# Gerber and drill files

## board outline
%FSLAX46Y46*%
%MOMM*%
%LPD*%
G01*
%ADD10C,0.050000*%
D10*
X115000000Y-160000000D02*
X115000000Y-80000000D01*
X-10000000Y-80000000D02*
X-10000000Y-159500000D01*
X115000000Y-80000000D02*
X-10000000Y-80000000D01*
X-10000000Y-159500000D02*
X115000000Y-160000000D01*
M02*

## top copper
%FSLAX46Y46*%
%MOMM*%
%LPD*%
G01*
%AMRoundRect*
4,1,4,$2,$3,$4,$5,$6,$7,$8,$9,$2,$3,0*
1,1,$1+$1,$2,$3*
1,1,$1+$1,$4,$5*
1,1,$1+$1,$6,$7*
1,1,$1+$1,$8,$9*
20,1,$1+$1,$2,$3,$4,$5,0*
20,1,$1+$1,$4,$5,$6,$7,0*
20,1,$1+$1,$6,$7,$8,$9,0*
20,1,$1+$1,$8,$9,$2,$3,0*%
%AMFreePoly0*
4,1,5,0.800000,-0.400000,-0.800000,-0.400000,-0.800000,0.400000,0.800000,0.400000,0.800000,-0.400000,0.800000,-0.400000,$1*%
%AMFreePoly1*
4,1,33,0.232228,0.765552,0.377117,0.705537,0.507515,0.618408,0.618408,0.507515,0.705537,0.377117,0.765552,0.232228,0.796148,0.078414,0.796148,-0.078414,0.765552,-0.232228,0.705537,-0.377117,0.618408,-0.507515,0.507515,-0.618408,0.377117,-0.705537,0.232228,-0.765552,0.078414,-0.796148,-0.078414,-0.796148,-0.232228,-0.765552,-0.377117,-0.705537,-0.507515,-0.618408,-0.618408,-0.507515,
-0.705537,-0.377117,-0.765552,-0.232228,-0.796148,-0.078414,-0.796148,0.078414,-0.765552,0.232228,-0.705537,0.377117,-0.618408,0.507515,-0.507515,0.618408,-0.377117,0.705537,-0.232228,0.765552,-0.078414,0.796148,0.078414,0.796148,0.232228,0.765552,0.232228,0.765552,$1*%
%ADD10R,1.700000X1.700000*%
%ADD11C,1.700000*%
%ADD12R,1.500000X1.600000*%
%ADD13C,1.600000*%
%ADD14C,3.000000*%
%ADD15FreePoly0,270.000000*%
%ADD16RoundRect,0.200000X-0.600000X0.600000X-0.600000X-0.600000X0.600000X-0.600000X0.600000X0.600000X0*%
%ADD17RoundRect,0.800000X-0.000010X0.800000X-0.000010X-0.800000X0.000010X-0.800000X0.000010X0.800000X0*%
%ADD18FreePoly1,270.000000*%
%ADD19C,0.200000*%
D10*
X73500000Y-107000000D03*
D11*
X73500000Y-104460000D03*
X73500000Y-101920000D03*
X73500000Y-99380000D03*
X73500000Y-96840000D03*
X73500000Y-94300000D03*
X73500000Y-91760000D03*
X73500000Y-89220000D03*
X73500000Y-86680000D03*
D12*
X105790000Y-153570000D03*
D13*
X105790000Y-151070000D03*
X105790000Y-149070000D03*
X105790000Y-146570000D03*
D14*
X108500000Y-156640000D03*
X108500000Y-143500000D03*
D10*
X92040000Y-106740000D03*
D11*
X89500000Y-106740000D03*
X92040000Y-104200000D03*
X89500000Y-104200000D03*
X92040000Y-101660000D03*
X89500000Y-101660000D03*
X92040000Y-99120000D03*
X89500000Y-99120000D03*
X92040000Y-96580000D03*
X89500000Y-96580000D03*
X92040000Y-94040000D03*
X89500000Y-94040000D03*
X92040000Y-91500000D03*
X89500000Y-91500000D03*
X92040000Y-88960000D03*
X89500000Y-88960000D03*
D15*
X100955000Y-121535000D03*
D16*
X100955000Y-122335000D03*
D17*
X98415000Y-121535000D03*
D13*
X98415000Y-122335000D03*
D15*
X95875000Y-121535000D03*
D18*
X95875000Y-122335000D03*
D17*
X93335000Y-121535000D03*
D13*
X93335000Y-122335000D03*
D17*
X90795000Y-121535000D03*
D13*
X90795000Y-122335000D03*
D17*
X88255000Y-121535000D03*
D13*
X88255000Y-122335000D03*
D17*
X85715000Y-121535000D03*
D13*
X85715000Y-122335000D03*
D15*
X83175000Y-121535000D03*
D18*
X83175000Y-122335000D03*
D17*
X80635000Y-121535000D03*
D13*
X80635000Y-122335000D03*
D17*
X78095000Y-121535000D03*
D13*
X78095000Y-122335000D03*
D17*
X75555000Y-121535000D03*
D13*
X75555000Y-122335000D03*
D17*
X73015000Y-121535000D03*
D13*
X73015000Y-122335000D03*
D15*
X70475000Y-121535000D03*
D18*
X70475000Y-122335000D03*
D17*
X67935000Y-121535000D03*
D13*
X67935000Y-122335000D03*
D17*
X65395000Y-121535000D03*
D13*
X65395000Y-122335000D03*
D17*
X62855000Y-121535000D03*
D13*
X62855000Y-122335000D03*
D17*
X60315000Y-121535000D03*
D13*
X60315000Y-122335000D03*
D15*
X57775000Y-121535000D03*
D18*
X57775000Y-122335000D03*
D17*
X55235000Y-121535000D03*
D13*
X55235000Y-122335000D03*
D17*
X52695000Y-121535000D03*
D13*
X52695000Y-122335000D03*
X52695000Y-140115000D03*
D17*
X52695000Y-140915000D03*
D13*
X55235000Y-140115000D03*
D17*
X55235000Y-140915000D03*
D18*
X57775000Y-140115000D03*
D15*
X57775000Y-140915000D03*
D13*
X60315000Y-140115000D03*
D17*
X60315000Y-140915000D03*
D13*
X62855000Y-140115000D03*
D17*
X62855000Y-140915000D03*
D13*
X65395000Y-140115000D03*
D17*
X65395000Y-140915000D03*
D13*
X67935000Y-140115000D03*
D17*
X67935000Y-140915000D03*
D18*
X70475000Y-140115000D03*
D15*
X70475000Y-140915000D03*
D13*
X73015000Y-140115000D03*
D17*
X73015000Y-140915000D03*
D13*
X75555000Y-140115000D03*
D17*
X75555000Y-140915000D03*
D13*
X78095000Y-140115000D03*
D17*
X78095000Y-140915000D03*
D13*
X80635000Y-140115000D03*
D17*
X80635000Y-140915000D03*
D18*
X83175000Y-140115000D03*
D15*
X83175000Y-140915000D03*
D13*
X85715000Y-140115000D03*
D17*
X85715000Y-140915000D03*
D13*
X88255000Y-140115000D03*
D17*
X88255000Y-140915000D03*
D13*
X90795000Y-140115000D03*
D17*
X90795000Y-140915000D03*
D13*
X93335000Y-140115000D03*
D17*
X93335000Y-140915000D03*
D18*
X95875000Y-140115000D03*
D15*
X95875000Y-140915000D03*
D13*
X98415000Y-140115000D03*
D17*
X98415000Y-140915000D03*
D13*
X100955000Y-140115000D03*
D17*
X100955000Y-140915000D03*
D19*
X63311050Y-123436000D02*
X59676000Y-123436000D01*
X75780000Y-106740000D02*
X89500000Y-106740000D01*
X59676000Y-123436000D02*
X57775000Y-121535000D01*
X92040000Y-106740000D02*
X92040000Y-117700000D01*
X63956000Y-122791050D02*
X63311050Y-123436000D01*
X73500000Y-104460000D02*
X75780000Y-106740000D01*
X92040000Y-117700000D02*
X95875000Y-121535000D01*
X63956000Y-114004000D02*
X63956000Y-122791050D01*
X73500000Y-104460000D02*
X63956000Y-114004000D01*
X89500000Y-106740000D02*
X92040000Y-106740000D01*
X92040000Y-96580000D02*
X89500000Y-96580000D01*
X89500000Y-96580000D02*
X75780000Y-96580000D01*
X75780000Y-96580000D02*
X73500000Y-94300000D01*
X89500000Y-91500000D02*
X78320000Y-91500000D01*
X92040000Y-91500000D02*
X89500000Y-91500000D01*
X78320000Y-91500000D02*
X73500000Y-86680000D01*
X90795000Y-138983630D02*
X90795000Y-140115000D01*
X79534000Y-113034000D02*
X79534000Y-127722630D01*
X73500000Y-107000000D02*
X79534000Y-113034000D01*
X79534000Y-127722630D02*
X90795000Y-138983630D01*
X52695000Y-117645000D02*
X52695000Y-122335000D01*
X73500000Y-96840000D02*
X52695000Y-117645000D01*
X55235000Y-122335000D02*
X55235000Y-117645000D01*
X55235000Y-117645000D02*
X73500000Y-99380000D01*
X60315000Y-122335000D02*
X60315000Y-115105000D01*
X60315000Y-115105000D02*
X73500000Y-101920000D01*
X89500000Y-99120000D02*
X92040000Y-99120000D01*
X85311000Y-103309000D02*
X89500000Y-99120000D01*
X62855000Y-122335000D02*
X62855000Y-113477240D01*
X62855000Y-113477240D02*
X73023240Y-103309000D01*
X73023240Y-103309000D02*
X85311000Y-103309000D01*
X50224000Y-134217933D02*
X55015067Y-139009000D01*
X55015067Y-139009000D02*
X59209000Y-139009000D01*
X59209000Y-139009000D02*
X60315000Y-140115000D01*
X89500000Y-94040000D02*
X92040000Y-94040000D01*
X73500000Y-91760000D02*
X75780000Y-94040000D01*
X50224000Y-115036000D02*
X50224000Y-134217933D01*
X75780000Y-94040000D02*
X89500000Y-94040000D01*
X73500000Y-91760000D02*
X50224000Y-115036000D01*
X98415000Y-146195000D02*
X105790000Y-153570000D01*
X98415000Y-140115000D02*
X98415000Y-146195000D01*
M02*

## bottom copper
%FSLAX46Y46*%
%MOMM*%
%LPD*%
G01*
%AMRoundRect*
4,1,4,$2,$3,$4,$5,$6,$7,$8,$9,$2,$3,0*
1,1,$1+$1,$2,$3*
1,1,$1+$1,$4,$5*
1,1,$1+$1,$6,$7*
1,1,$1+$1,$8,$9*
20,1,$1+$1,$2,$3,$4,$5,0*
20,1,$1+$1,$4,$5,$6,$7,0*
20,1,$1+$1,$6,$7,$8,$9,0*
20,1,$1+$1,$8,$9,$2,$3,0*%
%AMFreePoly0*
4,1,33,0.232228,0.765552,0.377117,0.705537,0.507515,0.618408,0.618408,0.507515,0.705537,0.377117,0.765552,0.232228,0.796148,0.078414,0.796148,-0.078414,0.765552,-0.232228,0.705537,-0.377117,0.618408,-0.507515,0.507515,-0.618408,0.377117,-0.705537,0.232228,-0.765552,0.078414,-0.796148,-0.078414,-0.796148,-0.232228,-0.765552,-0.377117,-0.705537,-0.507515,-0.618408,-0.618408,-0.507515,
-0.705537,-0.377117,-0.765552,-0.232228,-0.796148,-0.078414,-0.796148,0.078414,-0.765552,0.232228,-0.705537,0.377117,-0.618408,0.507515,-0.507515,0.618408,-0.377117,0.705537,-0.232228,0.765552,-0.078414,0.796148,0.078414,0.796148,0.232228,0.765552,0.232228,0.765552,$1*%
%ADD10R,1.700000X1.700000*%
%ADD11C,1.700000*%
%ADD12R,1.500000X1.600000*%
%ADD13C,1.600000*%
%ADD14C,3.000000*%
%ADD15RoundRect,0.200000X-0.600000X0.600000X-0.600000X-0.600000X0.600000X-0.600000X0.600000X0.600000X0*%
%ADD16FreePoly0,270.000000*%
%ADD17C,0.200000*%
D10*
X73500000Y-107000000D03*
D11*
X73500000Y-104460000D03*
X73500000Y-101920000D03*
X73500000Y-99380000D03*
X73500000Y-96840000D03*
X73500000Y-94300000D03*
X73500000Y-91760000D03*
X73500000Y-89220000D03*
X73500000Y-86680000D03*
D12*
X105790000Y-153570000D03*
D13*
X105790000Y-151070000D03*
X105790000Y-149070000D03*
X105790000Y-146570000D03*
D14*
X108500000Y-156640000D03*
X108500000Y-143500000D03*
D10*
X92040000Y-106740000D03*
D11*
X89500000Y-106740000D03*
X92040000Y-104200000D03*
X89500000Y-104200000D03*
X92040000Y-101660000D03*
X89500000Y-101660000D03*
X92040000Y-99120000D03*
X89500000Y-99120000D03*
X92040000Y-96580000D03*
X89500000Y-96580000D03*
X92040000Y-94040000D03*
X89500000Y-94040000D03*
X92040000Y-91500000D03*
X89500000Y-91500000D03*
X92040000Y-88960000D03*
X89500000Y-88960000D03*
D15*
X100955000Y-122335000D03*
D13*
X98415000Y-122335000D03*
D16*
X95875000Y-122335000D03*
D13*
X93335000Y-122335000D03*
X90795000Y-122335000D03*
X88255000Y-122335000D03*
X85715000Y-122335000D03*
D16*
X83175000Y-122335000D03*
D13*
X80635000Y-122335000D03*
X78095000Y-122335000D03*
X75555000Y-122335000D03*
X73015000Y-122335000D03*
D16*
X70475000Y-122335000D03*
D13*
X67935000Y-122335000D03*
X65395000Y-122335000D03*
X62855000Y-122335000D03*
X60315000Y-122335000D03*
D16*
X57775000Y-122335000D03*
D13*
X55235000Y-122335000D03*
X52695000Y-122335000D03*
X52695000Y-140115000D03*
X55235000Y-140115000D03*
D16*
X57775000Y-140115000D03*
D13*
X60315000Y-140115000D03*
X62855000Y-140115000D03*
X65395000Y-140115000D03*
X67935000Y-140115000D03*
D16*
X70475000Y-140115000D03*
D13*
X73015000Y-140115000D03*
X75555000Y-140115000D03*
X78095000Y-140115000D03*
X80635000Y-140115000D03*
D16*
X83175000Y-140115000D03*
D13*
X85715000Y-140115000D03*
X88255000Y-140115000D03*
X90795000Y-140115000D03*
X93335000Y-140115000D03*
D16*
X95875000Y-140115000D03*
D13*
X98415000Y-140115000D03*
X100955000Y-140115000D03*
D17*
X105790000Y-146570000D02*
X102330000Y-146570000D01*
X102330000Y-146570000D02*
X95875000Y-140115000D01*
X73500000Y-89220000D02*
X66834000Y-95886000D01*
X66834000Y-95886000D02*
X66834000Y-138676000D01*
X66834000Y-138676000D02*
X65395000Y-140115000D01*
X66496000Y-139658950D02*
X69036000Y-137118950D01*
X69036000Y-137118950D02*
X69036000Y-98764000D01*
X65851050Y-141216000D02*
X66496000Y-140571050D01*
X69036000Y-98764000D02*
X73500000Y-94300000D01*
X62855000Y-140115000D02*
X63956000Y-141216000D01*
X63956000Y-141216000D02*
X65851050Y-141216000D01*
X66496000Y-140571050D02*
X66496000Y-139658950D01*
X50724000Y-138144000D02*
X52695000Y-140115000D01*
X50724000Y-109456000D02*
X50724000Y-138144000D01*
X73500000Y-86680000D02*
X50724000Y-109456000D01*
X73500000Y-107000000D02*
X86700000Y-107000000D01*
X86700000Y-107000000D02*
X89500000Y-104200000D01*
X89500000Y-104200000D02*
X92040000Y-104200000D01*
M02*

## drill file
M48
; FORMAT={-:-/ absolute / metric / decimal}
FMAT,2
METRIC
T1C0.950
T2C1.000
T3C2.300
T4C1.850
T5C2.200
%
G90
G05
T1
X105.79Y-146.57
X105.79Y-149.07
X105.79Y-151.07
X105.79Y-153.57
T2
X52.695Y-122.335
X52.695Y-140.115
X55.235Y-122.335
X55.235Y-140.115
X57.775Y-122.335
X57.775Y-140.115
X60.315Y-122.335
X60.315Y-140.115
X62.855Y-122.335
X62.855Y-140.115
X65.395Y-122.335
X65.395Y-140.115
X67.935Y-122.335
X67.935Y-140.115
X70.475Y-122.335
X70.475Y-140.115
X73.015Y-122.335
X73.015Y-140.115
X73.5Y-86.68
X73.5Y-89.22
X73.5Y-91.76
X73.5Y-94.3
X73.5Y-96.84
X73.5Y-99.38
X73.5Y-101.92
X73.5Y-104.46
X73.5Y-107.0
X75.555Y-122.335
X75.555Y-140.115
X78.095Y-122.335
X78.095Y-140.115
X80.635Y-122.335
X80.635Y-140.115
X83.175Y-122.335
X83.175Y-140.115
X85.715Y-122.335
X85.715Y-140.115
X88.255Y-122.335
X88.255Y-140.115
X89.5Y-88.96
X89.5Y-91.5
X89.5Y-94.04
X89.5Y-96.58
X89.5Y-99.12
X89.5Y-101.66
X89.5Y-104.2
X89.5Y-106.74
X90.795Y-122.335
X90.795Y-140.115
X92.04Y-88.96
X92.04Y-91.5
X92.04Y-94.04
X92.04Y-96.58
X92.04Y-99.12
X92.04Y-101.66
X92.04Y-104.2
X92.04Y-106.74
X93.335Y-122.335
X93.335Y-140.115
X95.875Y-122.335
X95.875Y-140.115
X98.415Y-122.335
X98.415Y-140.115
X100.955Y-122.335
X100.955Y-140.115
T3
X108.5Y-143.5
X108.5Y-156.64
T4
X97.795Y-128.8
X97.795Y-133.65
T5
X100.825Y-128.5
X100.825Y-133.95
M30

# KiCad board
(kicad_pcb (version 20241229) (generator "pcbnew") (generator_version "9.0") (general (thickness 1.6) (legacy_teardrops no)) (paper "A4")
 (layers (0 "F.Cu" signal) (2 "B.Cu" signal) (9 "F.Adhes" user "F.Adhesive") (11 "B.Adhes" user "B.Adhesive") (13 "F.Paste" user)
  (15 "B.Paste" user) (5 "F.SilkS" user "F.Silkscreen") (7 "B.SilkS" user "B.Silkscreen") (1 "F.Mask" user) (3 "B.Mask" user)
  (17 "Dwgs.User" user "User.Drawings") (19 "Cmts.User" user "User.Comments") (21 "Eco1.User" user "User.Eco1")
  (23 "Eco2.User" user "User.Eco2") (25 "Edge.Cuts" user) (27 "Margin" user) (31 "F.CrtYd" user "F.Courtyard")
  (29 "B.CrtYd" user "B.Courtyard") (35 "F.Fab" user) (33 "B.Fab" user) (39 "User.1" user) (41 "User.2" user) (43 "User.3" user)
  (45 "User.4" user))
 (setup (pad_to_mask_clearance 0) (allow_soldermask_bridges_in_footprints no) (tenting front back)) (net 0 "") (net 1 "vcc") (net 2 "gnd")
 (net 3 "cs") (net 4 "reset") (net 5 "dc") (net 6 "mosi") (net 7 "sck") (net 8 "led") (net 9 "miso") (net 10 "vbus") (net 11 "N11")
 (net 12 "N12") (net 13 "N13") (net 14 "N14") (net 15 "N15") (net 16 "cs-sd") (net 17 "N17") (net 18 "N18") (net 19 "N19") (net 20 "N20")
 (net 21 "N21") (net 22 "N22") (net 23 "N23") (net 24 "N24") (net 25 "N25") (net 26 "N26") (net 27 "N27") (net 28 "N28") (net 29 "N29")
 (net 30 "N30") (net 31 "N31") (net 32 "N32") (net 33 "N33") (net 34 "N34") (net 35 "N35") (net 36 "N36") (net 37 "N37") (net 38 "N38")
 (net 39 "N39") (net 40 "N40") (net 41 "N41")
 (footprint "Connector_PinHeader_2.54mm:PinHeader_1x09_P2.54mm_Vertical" (layer "F.Cu") (at 73.5 107 180)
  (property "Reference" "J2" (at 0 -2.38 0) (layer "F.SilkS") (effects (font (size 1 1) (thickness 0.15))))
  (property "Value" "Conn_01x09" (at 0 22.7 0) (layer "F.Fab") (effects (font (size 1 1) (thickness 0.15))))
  (pad "1" thru_hole rect (at 0 0 180) (size 1.7 1.7) (drill 1) (layers "*.Cu" "*.Mask") (remove_unused_layers no) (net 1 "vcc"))
  (pad "2" thru_hole circle (at 0 2.54 180) (size 1.7 1.7) (drill 1) (layers "*.Cu" "*.Mask") (remove_unused_layers no) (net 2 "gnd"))
  (pad "3" thru_hole circle (at 0 5.08 180) (size 1.7 1.7) (drill 1) (layers "*.Cu" "*.Mask") (remove_unused_layers no) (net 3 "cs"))
  (pad "4" thru_hole circle (at 0 7.62 180) (size 1.7 1.7) (drill 1) (layers "*.Cu" "*.Mask") (remove_unused_layers no) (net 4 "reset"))
  (pad "5" thru_hole circle (at 0 10.16 180) (size 1.7 1.7) (drill 1) (layers "*.Cu" "*.Mask") (remove_unused_layers no) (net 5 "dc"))
  (pad "6" thru_hole circle (at 0 12.7 180) (size 1.7 1.7) (drill 1) (layers "*.Cu" "*.Mask") (remove_unused_layers no) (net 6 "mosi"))
  (pad "7" thru_hole circle (at 0 15.24 180) (size 1.7 1.7) (drill 1) (layers "*.Cu" "*.Mask") (remove_unused_layers no) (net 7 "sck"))
  (pad "8" thru_hole circle (at 0 17.78 180) (size 1.7 1.7) (drill 1) (layers "*.Cu" "*.Mask") (remove_unused_layers no) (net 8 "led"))
  (pad "9" thru_hole circle (at 0 20.32 180) (size 1.7 1.7) (drill 1) (layers "*.Cu" "*.Mask") (remove_unused_layers no) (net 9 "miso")))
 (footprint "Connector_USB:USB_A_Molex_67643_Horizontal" (layer "F.Cu") (at 105.79 153.57 90)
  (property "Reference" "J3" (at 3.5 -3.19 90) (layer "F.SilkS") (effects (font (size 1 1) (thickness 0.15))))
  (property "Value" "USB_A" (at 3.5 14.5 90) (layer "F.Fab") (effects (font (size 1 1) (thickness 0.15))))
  (pad "1" thru_hole rect (at 0 0 90) (size 1.6 1.5) (drill 0.95) (layers "*.Cu" "*.Mask") (remove_unused_layers no) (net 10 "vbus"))
  (pad "2" thru_hole circle (at 2.5 0 90) (size 1.6 1.6) (drill 0.95) (layers "*.Cu" "*.Mask") (remove_unused_layers no) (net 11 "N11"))
  (pad "3" thru_hole circle (at 4.5 0 90) (size 1.6 1.6) (drill 0.95) (layers "*.Cu" "*.Mask") (remove_unused_layers no) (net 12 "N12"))
  (pad "4" thru_hole circle (at 7 0 90) (size 1.6 1.6) (drill 0.95) (layers "*.Cu" "*.Mask") (remove_unused_layers no) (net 2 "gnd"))
  (pad "5" thru_hole circle (at -3.07 2.71 90) (size 3 3) (drill 2.3) (layers "*.Cu" "*.Mask") (remove_unused_layers no) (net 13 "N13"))
  (pad "5" thru_hole circle (at 10.07 2.71 90) (size 3 3) (drill 2.3) (layers "*.Cu" "*.Mask") (remove_unused_layers no) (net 13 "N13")))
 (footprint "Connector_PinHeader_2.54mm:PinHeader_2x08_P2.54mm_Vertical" (layer "F.Cu") (at 92.04 106.74 180)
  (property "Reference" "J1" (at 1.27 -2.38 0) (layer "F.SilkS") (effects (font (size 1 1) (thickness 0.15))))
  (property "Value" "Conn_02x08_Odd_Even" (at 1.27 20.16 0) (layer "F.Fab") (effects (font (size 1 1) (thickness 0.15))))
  (pad "1" thru_hole rect (at 0 0 180) (size 1.7 1.7) (drill 1) (layers "*.Cu" "*.Mask") (remove_unused_layers no) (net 2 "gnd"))
  (pad "2" thru_hole circle (at 2.54 0 180) (size 1.7 1.7) (drill 1) (layers "*.Cu" "*.Mask") (remove_unused_layers no) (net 2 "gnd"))
  (pad "3" thru_hole circle (at 0 2.54 180) (size 1.7 1.7) (drill 1) (layers "*.Cu" "*.Mask") (remove_unused_layers no) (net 1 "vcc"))
  (pad "4" thru_hole circle (at 2.54 2.54 180) (size 1.7 1.7) (drill 1) (layers "*.Cu" "*.Mask") (remove_unused_layers no) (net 1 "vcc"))
  (pad "5" thru_hole circle (at 0 5.08 180) (size 1.7 1.7) (drill 1) (layers "*.Cu" "*.Mask") (remove_unused_layers no) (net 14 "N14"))
  (pad "6" thru_hole circle (at 2.54 5.08 180) (size 1.7 1.7) (drill 1) (layers "*.Cu" "*.Mask") (remove_unused_layers no) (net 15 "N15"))
  (pad "7" thru_hole circle (at 0 7.62 180) (size 1.7 1.7) (drill 1) (layers "*.Cu" "*.Mask") (remove_unused_layers no) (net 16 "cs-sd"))
  (pad "8" thru_hole circle (at 2.54 7.62 180) (size 1.7 1.7) (drill 1) (layers "*.Cu" "*.Mask") (remove_unused_layers no) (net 16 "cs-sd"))
  (pad "9" thru_hole circle (at 0 10.16 180) (size 1.7 1.7) (drill 1) (layers "*.Cu" "*.Mask") (remove_unused_layers no) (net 6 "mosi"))
  (pad "10" thru_hole circle (at 2.54 10.16 180) (size 1.7 1.7) (drill 1) (layers "*.Cu" "*.Mask") (remove_unused_layers no) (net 6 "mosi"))
  (pad "11" thru_hole circle (at 0 12.7 180) (size 1.7 1.7) (drill 1) (layers "*.Cu" "*.Mask") (remove_unused_layers no) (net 7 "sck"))
  (pad "12" thru_hole circle (at 2.54 12.7 180) (size 1.7 1.7) (drill 1) (layers "*.Cu" "*.Mask") (remove_unused_layers no) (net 7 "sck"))
  (pad "13" thru_hole circle (at 0 15.24 180) (size 1.7 1.7) (drill 1) (layers "*.Cu" "*.Mask") (remove_unused_layers no) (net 9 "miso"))
  (pad "14" thru_hole circle (at 2.54 15.24 180) (size 1.7 1.7) (drill 1) (layers "*.Cu" "*.Mask") (remove_unused_layers no) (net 9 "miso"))
  (pad "15" thru_hole circle (at 0 17.78 180) (size 1.7 1.7) (drill 1) (layers "*.Cu" "*.Mask") (remove_unused_layers no) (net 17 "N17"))
  (pad "16" thru_hole circle (at 2.54 17.78 180) (size 1.7 1.7) (drill 1) (layers "*.Cu" "*.Mask") (remove_unused_layers no) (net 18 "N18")))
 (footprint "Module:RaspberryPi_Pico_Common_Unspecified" (layer "F.Cu") (at 76.825 131.225 -90)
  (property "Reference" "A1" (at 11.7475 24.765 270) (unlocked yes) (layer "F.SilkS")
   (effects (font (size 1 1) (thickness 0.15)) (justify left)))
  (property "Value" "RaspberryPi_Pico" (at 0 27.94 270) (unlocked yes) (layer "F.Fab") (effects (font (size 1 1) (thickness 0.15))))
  (pad "" np_thru_hole circle (at -2.725 -24 270) (size 2.2 2.2) (drill 2.2) (layers "*.Mask"))
  (pad "" np_thru_hole circle (at -2.425 -20.97 270) (size 1.85 1.85) (drill 1.85) (layers "*.Mask"))
  (pad "" np_thru_hole circle (at 2.425 -20.97 270) (size 1.85 1.85) (drill 1.85) (layers "*.Mask"))
  (pad "" np_thru_hole circle (at 2.725 -24 270) (size 2.2 2.2) (drill 2.2) (layers "*.Mask"))
  (pad "1" smd custom (at -9.69 -24.13 270) (size 1.6 0.8) (layers "F.Cu" "F.Mask") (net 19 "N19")
   (options (clearance outline) (anchor rect)) (primitives))
  (pad "1" thru_hole roundrect (at -8.89 -24.13 270) (size 1.6 1.6) (drill 1) (layers "*.Cu" "*.Mask") (remove_unused_layers no)
   (roundrect_rratio 0.125) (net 19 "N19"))
  (pad "2" smd roundrect (at -9.69 -21.59 270) (size 3.2 1.6) (layers "F.Cu" "F.Mask") (roundrect_rratio 0.5) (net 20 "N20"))
  (pad "2" thru_hole circle (at -8.89 -21.59 270) (size 1.6 1.6) (drill 1) (layers "*.Cu" "*.Mask") (remove_unused_layers no) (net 20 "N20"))
  (pad "3" smd custom (at -9.69 -19.05 270) (size 1.6 0.8) (layers "F.Cu" "F.Mask") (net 2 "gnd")
   (options (clearance outline) (anchor rect)) (primitives))
  (pad "3" thru_hole custom (at -8.89 -19.05 270) (size 1.6 1.6) (drill 1) (layers "*.Cu" "*.Mask") (remove_unused_layers no) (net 2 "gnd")
   (options (clearance outline) (anchor circle)) (primitives))
  (pad "4" smd roundrect (at -9.69 -16.51 270) (size 3.2 1.6) (layers "F.Cu" "F.Mask") (roundrect_rratio 0.5) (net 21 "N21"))
  (pad "4" thru_hole circle (at -8.89 -16.51 270) (size 1.6 1.6) (drill 1) (layers "*.Cu" "*.Mask") (remove_unused_layers no) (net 21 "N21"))
  (pad "5" smd roundrect (at -9.69 -13.97 270) (size 3.2 1.6) (layers "F.Cu" "F.Mask") (roundrect_rratio 0.5) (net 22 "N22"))
  (pad "5" thru_hole circle (at -8.89 -13.97 270) (size 1.6 1.6) (drill 1) (layers "*.Cu" "*.Mask") (remove_unused_layers no) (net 22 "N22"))
  (pad "6" smd roundrect (at -9.69 -11.43 270) (size 3.2 1.6) (layers "F.Cu" "F.Mask") (roundrect_rratio 0.5) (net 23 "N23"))
  (pad "6" thru_hole circle (at -8.89 -11.43 270) (size 1.6 1.6) (drill 1) (layers "*.Cu" "*.Mask") (remove_unused_layers no) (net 23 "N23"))
  (pad "7" smd roundrect (at -9.69 -8.89 270) (size 3.2 1.6) (layers "F.Cu" "F.Mask") (roundrect_rratio 0.5) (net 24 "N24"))
  (pad "7" thru_hole circle (at -8.89 -8.89 270) (size 1.6 1.6) (drill 1) (layers "*.Cu" "*.Mask") (remove_unused_layers no) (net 24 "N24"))
  (pad "8" smd custom (at -9.69 -6.35 270) (size 1.6 0.8) (layers "F.Cu" "F.Mask") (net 2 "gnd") (options (clearance outline) (anchor rect))
   (primitives))
  (pad "8" thru_hole custom (at -8.89 -6.35 270) (size 1.6 1.6) (drill 1) (layers "*.Cu" "*.Mask") (remove_unused_layers no) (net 2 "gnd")
   (options (clearance outline) (anchor circle)) (primitives))
  (pad "9" smd roundrect (at -9.69 -3.81 270) (size 3.2 1.6) (layers "F.Cu" "F.Mask") (roundrect_rratio 0.5) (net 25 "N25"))
  (pad "9" thru_hole circle (at -8.89 -3.81 270) (size 1.6 1.6) (drill 1) (layers "*.Cu" "*.Mask") (remove_unused_layers no) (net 25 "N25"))
  (pad "10" smd roundrect (at -9.69 -1.27 270) (size 3.2 1.6) (layers "F.Cu" "F.Mask") (roundrect_rratio 0.5) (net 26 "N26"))
  (pad "10" thru_hole circle (at -8.89 -1.27 270) (size 1.6 1.6) (drill 1) (layers "*.Cu" "*.Mask") (remove_unused_layers no) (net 26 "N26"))
  (pad "11" smd roundrect (at -9.69 1.27 270) (size 3.2 1.6) (layers "F.Cu" "F.Mask") (roundrect_rratio 0.5) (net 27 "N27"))
  (pad "11" thru_hole circle (at -8.89 1.27 270) (size 1.6 1.6) (drill 1) (layers "*.Cu" "*.Mask") (remove_unused_layers no) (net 27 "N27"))
  (pad "12" smd roundrect (at -9.69 3.81 270) (size 3.2 1.6) (layers "F.Cu" "F.Mask") (roundrect_rratio 0.5) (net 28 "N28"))
  (pad "12" thru_hole circle (at -8.89 3.81 270) (size 1.6 1.6) (drill 1) (layers "*.Cu" "*.Mask") (remove_unused_layers no) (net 28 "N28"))
  (pad "13" smd custom (at -9.69 6.35 270) (size 1.6 0.8) (layers "F.Cu" "F.Mask") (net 2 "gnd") (options (clearance outline) (anchor rect))
   (primitives))
  (pad "13" thru_hole custom (at -8.89 6.35 270) (size 1.6 1.6) (drill 1) (layers "*.Cu" "*.Mask") (remove_unused_layers no) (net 2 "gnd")
   (options (clearance outline) (anchor circle)) (primitives))
  (pad "14" smd roundrect (at -9.69 8.89 270) (size 3.2 1.6) (layers "F.Cu" "F.Mask") (roundrect_rratio 0.5) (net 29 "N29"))
  (pad "14" thru_hole circle (at -8.89 8.89 270) (size 1.6 1.6) (drill 1) (layers "*.Cu" "*.Mask") (remove_unused_layers no) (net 29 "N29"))
  (pad "15" smd roundrect (at -9.69 11.43 270) (size 3.2 1.6) (layers "F.Cu" "F.Mask") (roundrect_rratio 0.5) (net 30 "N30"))
  (pad "15" thru_hole circle (at -8.89 11.43 270) (size 1.6 1.6) (drill 1) (layers "*.Cu" "*.Mask") (remove_unused_layers no) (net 30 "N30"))
  (pad "16" smd roundrect (at -9.69 13.97 270) (size 3.2 1.6) (layers "F.Cu" "F.Mask") (roundrect_rratio 0.5) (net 16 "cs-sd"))
  (pad "16" thru_hole circle (at -8.89 13.97 270) (size 1.6 1.6) (drill 1) (layers "*.Cu" "*.Mask") (remove_unused_layers no)
   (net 16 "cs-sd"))
  (pad "17" smd roundrect (at -9.69 16.51 270) (size 3.2 1.6) (layers "F.Cu" "F.Mask") (roundrect_rratio 0.5) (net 3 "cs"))
  (pad "17" thru_hole circle (at -8.89 16.51 270) (size 1.6 1.6) (drill 1) (layers "*.Cu" "*.Mask") (remove_unused_layers no) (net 3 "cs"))
  (pad "18" smd custom (at -9.69 19.05 270) (size 1.6 0.8) (layers "F.Cu" "F.Mask") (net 2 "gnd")
   (options (clearance outline) (anchor rect)) (primitives))
  (pad "18" thru_hole custom (at -8.89 19.05 270) (size 1.6 1.6) (drill 1) (layers "*.Cu" "*.Mask") (remove_unused_layers no) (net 2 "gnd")
   (options (clearance outline) (anchor circle)) (primitives))
  (pad "19" smd roundrect (at -9.69 21.59 270) (size 3.2 1.6) (layers "F.Cu" "F.Mask") (roundrect_rratio 0.5) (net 4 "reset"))
  (pad "19" thru_hole circle (at -8.89 21.59 270) (size 1.6 1.6) (drill 1) (layers "*.Cu" "*.Mask") (remove_unused_layers no)
   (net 4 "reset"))
  (pad "20" smd roundrect (at -9.69 24.13 270) (size 3.2 1.6) (layers "F.Cu" "F.Mask") (roundrect_rratio 0.5) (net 5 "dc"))
  (pad "20" thru_hole circle (at -8.89 24.13 270) (size 1.6 1.6) (drill 1) (layers "*.Cu" "*.Mask") (remove_unused_layers no) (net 5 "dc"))
  (pad "21" thru_hole circle (at 8.89 24.13 270) (size 1.6 1.6) (drill 1) (layers "*.Cu" "*.Mask") (remove_unused_layers no) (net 9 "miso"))
  (pad "21" smd roundrect (at 9.69 24.13 270) (size 3.2 1.6) (layers "F.Cu" "F.Mask") (roundrect_rratio 0.5) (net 9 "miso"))
  (pad "22" thru_hole circle (at 8.89 21.59 270) (size 1.6 1.6) (drill 1) (layers "*.Cu" "*.Mask") (remove_unused_layers no) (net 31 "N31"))
  (pad "22" smd roundrect (at 9.69 21.59 270) (size 3.2 1.6) (layers "F.Cu" "F.Mask") (roundrect_rratio 0.5) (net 31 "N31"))
  (pad "23" thru_hole custom (at 8.89 19.05 270) (size 1.6 1.6) (drill 1) (layers "*.Cu" "*.Mask") (remove_unused_layers no) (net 2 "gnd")
   (options (clearance outline) (anchor circle)) (primitives))
  (pad "23" smd custom (at 9.69 19.05 270) (size 1.6 0.8) (layers "F.Cu" "F.Mask") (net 2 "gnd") (options (clearance outline) (anchor rect))
   (primitives))
  (pad "24" thru_hole circle (at 8.89 16.51 270) (size 1.6 1.6) (drill 1) (layers "*.Cu" "*.Mask") (remove_unused_layers no) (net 7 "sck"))
  (pad "24" smd roundrect (at 9.69 16.51 270) (size 3.2 1.6) (layers "F.Cu" "F.Mask") (roundrect_rratio 0.5) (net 7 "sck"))
  (pad "25" thru_hole circle (at 8.89 13.97 270) (size 1.6 1.6) (drill 1) (layers "*.Cu" "*.Mask") (remove_unused_layers no) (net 6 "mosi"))
  (pad "25" smd roundrect (at 9.69 13.97 270) (size 3.2 1.6) (layers "F.Cu" "F.Mask") (roundrect_rratio 0.5) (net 6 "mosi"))
  (pad "26" thru_hole circle (at 8.89 11.43 270) (size 1.6 1.6) (drill 1) (layers "*.Cu" "*.Mask") (remove_unused_layers no) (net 8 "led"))
  (pad "26" smd roundrect (at 9.69 11.43 270) (size 3.2 1.6) (layers "F.Cu" "F.Mask") (roundrect_rratio 0.5) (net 8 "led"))
  (pad "27" thru_hole circle (at 8.89 8.89 270) (size 1.6 1.6) (drill 1) (layers "*.Cu" "*.Mask") (remove_unused_layers no) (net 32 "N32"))
  (pad "27" smd roundrect (at 9.69 8.89 270) (size 3.2 1.6) (layers "F.Cu" "F.Mask") (roundrect_rratio 0.5) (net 32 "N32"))
  (pad "28" thru_hole custom (at 8.89 6.35 270) (size 1.6 1.6) (drill 1) (layers "*.Cu" "*.Mask") (remove_unused_layers no) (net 2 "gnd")
   (options (clearance outline) (anchor circle)) (primitives))
  (pad "28" smd custom (at 9.69 6.35 270) (size 1.6 0.8) (layers "F.Cu" "F.Mask") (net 2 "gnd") (options (clearance outline) (anchor rect))
   (primitives))
  (pad "29" thru_hole circle (at 8.89 3.81 270) (size 1.6 1.6) (drill 1) (layers "*.Cu" "*.Mask") (remove_unused_layers no) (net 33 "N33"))
  (pad "29" smd roundrect (at 9.69 3.81 270) (size 3.2 1.6) (layers "F.Cu" "F.Mask") (roundrect_rratio 0.5) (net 33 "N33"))
  (pad "30" thru_hole circle (at 8.89 1.27 270) (size 1.6 1.6) (drill 1) (layers "*.Cu" "*.Mask") (remove_unused_layers no) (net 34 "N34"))
  (pad "30" smd roundrect (at 9.69 1.27 270) (size 3.2 1.6) (layers "F.Cu" "F.Mask") (roundrect_rratio 0.5) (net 34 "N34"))
  (pad "31" thru_hole circle (at 8.89 -1.27 270) (size 1.6 1.6) (drill 1) (layers "*.Cu" "*.Mask") (remove_unused_layers no) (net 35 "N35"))
  (pad "31" smd roundrect (at 9.69 -1.27 270) (size 3.2 1.6) (layers "F.Cu" "F.Mask") (roundrect_rratio 0.5) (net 35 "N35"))
  (pad "32" thru_hole circle (at 8.89 -3.81 270) (size 1.6 1.6) (drill 1) (layers "*.Cu" "*.Mask") (remove_unused_layers no) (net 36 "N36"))
  (pad "32" smd roundrect (at 9.69 -3.81 270) (size 3.2 1.6) (layers "F.Cu" "F.Mask") (roundrect_rratio 0.5) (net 36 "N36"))
  (pad "33" thru_hole custom (at 8.89 -6.35 270) (size 1.6 1.6) (drill 1) (layers "*.Cu" "*.Mask") (remove_unused_layers no) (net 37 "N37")
   (options (clearance outline) (anchor circle)) (primitives))
  (pad "33" smd custom (at 9.69 -6.35 270) (size 1.6 0.8) (layers "F.Cu" "F.Mask") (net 37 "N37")
   (options (clearance outline) (anchor rect)) (primitives))
  (pad "34" thru_hole circle (at 8.89 -8.89 270) (size 1.6 1.6) (drill 1) (layers "*.Cu" "*.Mask") (remove_unused_layers no) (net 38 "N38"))
  (pad "34" smd roundrect (at 9.69 -8.89 270) (size 3.2 1.6) (layers "F.Cu" "F.Mask") (roundrect_rratio 0.5) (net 38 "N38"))
  (pad "35" thru_hole circle (at 8.89 -11.43 270) (size 1.6 1.6) (drill 1) (layers "*.Cu" "*.Mask") (remove_unused_layers no) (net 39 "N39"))
  (pad "35" smd roundrect (at 9.69 -11.43 270) (size 3.2 1.6) (layers "F.Cu" "F.Mask") (roundrect_rratio 0.5) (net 39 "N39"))
  (pad "36" thru_hole circle (at 8.89 -13.97 270) (size 1.6 1.6) (drill 1) (layers "*.Cu" "*.Mask") (remove_unused_layers no) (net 1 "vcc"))
  (pad "36" smd roundrect (at 9.69 -13.97 270) (size 3.2 1.6) (layers "F.Cu" "F.Mask") (roundrect_rratio 0.5) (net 1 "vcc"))
  (pad "37" thru_hole circle (at 8.89 -16.51 270) (size 1.6 1.6) (drill 1) (layers "*.Cu" "*.Mask") (remove_unused_layers no) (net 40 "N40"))
  (pad "37" smd roundrect (at 9.69 -16.51 270) (size 3.2 1.6) (layers "F.Cu" "F.Mask") (roundrect_rratio 0.5) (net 40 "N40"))
  (pad "38" thru_hole custom (at 8.89 -19.05 270) (size 1.6 1.6) (drill 1) (layers "*.Cu" "*.Mask") (remove_unused_layers no) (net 2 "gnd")
   (options (clearance outline) (anchor circle)) (primitives))
  (pad "38" smd custom (at 9.69 -19.05 270) (size 1.6 0.8) (layers "F.Cu" "F.Mask") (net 2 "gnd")
   (options (clearance outline) (anchor rect)) (primitives))
  (pad "39" thru_hole circle (at 8.89 -21.59 270) (size 1.6 1.6) (drill 1) (layers "*.Cu" "*.Mask") (remove_unused_layers no)
   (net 10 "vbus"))
  (pad "39" smd roundrect (at 9.69 -21.59 270) (size 3.2 1.6) (layers "F.Cu" "F.Mask") (roundrect_rratio 0.5) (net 10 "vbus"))
  (pad "40" thru_hole circle (at 8.89 -24.13 270) (size 1.6 1.6) (drill 1) (layers "*.Cu" "*.Mask") (remove_unused_layers no) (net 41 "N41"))
  (pad "40" smd roundrect (at 9.69 -24.13 270) (size 3.2 1.6) (layers "F.Cu" "F.Mask") (roundrect_rratio 0.5) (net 41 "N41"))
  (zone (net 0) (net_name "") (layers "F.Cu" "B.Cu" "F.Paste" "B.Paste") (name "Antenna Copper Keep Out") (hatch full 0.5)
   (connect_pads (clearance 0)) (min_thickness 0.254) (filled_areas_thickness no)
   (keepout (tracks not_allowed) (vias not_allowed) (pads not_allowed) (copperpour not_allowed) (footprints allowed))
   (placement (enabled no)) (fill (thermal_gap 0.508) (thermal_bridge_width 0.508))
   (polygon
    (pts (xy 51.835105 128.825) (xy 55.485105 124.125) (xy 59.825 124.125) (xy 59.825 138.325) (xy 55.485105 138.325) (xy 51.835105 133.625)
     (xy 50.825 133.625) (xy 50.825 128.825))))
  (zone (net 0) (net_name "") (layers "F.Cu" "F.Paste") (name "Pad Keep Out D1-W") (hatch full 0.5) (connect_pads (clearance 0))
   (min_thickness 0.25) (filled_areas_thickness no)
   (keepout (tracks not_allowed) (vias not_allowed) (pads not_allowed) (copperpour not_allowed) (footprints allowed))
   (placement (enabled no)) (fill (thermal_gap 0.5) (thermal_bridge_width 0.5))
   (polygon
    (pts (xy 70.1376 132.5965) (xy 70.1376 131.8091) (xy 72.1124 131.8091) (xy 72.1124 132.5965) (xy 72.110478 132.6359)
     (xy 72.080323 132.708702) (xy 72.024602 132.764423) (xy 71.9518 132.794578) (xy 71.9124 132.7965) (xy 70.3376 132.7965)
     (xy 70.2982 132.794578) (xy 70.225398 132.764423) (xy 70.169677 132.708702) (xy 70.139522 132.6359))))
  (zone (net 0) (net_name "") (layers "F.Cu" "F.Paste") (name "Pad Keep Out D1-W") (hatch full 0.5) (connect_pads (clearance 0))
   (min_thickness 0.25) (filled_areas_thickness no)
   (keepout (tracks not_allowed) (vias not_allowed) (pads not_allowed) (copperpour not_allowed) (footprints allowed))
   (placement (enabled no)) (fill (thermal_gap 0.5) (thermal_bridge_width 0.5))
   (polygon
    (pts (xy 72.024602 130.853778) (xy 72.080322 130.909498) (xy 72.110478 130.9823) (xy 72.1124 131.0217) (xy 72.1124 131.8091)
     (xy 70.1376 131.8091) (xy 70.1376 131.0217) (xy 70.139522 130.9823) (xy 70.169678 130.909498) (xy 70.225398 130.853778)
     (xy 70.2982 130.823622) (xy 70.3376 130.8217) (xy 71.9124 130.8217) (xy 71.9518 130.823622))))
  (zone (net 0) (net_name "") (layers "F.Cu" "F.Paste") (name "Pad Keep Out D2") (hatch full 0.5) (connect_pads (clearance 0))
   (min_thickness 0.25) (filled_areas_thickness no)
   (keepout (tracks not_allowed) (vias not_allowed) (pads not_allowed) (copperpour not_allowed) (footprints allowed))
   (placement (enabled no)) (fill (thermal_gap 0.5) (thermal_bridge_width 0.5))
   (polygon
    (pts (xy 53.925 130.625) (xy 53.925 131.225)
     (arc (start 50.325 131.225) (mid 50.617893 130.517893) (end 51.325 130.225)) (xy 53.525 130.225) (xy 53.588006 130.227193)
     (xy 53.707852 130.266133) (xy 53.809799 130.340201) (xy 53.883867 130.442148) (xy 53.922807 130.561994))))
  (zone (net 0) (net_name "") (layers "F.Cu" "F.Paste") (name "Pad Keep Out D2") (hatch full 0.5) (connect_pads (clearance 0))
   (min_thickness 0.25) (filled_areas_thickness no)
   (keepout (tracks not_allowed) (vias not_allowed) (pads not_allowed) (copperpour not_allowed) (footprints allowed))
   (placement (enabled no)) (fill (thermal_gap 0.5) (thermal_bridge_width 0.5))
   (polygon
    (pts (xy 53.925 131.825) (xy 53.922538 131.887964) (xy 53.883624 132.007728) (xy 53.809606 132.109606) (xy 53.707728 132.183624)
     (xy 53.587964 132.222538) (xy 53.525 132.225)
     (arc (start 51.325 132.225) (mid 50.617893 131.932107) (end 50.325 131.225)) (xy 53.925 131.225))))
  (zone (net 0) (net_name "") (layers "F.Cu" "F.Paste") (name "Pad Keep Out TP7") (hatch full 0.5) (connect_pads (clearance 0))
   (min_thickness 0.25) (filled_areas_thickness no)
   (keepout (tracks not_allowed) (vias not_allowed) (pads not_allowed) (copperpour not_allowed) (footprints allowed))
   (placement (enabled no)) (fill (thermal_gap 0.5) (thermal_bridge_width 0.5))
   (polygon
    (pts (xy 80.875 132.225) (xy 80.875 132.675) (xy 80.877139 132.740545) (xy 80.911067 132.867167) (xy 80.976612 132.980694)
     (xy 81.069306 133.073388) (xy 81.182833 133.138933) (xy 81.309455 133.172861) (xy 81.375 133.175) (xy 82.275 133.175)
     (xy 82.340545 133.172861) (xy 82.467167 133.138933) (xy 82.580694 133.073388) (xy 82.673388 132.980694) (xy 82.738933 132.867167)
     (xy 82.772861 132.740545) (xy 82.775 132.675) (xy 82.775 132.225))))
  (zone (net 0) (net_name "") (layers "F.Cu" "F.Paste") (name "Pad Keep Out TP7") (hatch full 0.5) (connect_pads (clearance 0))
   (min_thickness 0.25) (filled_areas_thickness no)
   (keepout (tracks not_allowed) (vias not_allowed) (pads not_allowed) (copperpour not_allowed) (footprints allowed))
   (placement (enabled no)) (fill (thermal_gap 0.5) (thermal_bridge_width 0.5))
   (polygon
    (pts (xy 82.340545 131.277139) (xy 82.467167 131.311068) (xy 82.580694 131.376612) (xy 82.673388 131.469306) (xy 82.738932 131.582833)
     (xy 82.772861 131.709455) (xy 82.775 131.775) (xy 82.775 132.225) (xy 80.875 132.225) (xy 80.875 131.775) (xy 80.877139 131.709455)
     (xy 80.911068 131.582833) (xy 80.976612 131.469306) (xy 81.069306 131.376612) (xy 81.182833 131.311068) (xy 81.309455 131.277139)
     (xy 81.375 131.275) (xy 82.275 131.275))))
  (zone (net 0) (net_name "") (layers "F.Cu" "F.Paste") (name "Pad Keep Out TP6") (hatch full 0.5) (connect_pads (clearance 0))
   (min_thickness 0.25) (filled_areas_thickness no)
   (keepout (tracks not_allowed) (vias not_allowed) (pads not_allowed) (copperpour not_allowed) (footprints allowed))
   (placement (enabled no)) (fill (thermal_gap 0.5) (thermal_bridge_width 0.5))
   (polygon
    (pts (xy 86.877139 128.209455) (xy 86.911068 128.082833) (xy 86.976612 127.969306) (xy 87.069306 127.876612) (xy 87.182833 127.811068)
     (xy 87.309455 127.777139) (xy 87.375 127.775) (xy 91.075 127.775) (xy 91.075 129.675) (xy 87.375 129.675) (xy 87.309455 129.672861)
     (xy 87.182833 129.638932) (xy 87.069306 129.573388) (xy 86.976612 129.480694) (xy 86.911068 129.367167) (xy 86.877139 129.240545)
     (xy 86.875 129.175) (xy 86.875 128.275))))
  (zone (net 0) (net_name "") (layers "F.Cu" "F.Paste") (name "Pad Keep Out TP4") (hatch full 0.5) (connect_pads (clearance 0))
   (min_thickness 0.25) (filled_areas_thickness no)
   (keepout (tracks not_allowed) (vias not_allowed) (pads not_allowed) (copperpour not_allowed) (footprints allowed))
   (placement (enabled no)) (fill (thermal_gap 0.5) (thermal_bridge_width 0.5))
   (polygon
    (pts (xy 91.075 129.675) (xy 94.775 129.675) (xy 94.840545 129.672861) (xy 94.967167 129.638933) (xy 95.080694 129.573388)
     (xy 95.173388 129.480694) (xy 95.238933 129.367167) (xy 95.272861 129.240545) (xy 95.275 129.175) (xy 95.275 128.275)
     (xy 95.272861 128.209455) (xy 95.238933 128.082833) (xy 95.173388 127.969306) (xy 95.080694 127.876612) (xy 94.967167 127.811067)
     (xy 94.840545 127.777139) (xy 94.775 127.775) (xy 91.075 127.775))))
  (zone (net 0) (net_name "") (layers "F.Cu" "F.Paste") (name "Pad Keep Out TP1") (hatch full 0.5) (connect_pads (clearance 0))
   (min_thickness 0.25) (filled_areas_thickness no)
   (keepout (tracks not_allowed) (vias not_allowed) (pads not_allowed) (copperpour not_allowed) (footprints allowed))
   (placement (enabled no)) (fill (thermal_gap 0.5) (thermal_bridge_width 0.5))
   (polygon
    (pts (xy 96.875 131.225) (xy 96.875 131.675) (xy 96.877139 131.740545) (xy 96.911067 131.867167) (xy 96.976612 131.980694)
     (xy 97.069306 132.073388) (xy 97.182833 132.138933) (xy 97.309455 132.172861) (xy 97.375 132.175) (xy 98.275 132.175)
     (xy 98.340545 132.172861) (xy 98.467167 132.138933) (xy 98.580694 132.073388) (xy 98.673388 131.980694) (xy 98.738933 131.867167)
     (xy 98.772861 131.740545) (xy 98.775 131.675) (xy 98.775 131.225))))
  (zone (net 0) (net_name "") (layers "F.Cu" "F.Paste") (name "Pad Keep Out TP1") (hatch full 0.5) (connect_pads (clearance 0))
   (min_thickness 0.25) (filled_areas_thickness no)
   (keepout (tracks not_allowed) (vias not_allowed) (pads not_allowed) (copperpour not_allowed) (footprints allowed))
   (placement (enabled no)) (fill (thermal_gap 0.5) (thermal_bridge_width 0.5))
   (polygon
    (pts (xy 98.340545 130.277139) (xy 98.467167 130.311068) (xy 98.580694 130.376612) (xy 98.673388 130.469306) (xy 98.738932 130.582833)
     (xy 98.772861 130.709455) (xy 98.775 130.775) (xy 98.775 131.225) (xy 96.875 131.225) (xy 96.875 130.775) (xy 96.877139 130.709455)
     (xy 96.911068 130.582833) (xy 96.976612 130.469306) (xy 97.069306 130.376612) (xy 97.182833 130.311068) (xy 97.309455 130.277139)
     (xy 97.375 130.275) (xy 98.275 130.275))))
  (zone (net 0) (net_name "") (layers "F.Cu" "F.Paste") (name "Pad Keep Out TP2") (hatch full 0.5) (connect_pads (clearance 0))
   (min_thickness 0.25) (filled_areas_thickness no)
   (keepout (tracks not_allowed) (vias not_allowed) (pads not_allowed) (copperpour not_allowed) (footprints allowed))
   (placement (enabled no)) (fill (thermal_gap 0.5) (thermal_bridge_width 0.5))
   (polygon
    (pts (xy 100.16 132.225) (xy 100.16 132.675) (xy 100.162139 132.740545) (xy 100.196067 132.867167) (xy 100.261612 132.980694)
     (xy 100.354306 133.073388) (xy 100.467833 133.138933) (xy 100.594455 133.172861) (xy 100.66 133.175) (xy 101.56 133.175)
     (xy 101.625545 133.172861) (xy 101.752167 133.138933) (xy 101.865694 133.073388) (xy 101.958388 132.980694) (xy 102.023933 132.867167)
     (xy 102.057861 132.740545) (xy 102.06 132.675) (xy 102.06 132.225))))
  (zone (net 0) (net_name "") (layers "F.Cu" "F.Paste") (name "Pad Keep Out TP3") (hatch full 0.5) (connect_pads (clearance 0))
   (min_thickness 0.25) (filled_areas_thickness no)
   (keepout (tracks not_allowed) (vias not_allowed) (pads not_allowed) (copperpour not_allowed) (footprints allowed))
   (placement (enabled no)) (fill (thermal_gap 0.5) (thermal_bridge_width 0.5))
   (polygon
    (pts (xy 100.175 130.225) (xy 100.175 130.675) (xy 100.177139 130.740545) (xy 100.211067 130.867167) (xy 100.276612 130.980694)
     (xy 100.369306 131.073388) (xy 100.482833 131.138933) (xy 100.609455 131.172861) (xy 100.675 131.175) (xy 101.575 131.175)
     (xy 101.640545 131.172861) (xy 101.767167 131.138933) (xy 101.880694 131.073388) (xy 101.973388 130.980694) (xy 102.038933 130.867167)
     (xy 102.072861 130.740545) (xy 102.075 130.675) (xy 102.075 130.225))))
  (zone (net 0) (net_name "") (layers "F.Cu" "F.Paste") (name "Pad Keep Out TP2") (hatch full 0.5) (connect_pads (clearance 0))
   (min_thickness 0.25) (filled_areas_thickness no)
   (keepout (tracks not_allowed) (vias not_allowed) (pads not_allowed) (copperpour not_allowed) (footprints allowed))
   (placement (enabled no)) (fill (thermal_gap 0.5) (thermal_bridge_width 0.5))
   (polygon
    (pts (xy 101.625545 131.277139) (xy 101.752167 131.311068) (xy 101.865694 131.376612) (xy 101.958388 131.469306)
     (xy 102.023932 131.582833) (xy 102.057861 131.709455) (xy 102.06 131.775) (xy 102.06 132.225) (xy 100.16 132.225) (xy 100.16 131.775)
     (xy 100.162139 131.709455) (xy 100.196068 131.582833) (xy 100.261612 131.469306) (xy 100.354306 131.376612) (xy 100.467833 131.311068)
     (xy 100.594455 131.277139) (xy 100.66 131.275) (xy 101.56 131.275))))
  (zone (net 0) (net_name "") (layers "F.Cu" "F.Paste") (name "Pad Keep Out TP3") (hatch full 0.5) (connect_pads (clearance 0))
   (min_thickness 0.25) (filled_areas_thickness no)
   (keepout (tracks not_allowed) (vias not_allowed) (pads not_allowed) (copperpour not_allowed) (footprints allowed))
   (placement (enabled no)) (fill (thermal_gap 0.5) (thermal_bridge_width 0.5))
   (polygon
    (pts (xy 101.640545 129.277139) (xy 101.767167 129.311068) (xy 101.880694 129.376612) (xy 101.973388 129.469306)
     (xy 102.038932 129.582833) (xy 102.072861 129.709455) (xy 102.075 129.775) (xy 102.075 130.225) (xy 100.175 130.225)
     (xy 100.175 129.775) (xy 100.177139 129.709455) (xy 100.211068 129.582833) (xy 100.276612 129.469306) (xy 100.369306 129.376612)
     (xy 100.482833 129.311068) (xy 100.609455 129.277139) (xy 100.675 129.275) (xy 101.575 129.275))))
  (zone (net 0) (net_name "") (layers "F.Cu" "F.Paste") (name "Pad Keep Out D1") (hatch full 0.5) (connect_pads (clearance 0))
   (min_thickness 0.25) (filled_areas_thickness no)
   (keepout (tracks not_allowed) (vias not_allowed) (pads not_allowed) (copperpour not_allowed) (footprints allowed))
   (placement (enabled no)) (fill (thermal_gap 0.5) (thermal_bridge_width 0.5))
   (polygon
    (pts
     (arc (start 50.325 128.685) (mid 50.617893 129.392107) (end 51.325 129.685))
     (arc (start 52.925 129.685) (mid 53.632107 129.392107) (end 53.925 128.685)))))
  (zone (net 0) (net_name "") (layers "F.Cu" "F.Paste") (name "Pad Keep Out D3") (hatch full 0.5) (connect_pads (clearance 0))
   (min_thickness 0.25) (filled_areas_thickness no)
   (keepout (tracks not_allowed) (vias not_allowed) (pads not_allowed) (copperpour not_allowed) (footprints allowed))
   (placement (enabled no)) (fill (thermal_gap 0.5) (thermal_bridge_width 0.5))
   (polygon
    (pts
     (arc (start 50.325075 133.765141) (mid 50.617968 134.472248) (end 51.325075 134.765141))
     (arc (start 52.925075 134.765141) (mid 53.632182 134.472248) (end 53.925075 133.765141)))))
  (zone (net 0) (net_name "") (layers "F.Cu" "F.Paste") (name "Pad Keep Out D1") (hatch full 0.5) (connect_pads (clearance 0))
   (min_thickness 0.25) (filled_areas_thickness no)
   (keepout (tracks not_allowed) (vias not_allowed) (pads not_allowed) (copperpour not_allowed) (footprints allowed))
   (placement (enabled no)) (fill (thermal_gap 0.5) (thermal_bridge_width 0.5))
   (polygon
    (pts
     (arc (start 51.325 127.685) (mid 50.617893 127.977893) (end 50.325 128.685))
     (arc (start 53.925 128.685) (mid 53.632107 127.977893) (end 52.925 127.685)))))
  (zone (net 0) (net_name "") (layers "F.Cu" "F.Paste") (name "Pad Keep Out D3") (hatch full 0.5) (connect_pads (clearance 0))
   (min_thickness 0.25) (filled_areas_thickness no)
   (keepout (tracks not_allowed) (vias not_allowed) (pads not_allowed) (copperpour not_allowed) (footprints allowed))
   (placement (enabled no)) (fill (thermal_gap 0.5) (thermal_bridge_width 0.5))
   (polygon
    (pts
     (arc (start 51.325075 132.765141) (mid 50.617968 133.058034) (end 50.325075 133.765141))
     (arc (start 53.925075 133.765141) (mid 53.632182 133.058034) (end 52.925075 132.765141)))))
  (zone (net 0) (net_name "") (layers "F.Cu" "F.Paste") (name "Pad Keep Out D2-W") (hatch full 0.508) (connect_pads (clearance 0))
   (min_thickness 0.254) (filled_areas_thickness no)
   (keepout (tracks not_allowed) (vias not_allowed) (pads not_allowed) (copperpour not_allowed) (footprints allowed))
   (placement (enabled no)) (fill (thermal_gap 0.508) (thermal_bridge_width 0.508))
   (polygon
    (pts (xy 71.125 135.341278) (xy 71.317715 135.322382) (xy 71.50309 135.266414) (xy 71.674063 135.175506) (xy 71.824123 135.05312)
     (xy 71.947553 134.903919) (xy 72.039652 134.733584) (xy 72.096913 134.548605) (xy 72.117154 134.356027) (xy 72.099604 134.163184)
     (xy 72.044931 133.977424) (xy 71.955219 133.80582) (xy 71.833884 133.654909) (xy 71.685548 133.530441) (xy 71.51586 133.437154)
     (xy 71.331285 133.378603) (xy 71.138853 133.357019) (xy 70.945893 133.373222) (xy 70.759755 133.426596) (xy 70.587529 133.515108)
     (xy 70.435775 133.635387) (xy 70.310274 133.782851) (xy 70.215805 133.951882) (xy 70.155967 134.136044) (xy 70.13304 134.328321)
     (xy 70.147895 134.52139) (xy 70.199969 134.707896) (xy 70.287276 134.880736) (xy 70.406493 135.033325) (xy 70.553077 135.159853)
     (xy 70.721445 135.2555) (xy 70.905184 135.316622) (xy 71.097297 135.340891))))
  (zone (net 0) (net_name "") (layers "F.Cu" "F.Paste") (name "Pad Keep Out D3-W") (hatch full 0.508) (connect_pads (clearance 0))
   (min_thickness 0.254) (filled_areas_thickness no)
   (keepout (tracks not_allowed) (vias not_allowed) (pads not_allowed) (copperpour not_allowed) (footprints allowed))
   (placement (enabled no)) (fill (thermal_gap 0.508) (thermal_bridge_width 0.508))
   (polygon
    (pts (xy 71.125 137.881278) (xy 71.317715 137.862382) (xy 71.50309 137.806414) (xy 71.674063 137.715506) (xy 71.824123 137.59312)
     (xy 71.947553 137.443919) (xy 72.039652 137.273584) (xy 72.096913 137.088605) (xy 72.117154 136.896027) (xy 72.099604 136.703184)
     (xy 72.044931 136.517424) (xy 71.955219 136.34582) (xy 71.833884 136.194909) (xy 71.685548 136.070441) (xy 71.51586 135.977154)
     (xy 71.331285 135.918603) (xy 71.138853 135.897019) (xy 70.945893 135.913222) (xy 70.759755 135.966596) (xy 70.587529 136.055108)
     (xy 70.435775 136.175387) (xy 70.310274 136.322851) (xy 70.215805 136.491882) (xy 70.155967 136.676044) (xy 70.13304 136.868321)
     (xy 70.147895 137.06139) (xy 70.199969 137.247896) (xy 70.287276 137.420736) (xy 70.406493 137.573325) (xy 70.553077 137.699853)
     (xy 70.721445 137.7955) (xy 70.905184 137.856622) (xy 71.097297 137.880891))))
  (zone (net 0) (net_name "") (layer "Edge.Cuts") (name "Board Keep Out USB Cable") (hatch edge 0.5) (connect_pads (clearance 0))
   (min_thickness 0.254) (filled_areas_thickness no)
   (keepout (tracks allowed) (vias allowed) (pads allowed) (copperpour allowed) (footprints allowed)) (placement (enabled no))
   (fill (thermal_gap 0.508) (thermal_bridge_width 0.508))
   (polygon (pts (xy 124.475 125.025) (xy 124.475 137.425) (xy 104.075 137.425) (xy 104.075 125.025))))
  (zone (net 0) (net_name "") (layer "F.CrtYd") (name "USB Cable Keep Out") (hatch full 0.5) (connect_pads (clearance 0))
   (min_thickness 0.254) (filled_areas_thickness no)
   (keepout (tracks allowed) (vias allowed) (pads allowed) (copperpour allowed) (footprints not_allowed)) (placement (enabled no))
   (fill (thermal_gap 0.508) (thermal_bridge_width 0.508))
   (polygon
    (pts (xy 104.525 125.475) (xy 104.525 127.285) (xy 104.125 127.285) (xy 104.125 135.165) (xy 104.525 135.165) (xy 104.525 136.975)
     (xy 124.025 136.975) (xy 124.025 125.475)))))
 (gr_line (start 115 160) (end 115 80) (stroke (width 0.05) (type default)) (layer "Edge.Cuts"))
 (gr_line (start -10 80) (end -10 159.5) (stroke (width 0.05) (type default)) (layer "Edge.Cuts"))
 (gr_line (start 115 80) (end -10 80) (stroke (width 0.05) (type default)) (layer "Edge.Cuts"))
 (gr_line (start -10 159.5) (end 115 160) (stroke (width 0.05) (type default)) (layer "Edge.Cuts"))
 (segment (start 63.31105 123.436) (end 59.676 123.436) (width 0.2) (layer "F.Cu") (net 2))
 (segment (start 75.78 106.74) (end 89.5 106.74) (width 0.2) (layer "F.Cu") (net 2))
 (segment (start 59.676 123.436) (end 57.775 121.535) (width 0.2) (layer "F.Cu") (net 2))
 (segment (start 92.04 106.74) (end 92.04 117.7) (width 0.2) (layer "F.Cu") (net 2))
 (segment (start 63.956 122.79105) (end 63.31105 123.436) (width 0.2) (layer "F.Cu") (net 2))
 (segment (start 73.5 104.46) (end 75.78 106.74) (width 0.2) (layer "F.Cu") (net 2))
 (segment (start 92.04 117.7) (end 95.875 121.535) (width 0.2) (layer "F.Cu") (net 2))
 (segment (start 63.956 114.004) (end 63.956 122.79105) (width 0.2) (layer "F.Cu") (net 2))
 (segment (start 73.5 104.46) (end 63.956 114.004) (width 0.2) (layer "F.Cu") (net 2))
 (segment (start 89.5 106.74) (end 92.04 106.74) (width 0.2) (layer "F.Cu") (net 2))
 (segment (start 105.79 146.57) (end 102.33 146.57) (width 0.2) (layer "B.Cu") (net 2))
 (segment (start 102.33 146.57) (end 95.875 140.115) (width 0.2) (layer "B.Cu") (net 2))
 (segment (start 73.5 89.22) (end 66.834 95.886) (width 0.2) (layer "B.Cu") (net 8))
 (segment (start 66.834 95.886) (end 66.834 138.676) (width 0.2) (layer "B.Cu") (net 8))
 (segment (start 66.834 138.676) (end 65.395 140.115) (width 0.2) (layer "B.Cu") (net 8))
 (segment (start 92.04 96.58) (end 89.5 96.58) (width 0.2) (layer "F.Cu") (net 6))
 (segment (start 89.5 96.58) (end 75.78 96.58) (width 0.2) (layer "F.Cu") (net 6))
 (segment (start 75.78 96.58) (end 73.5 94.3) (width 0.2) (layer "F.Cu") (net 6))
 (segment (start 66.496 139.65895) (end 69.036 137.11895) (width 0.2) (layer "B.Cu") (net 6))
 (segment (start 69.036 137.11895) (end 69.036 98.764) (width 0.2) (layer "B.Cu") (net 6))
 (segment (start 65.85105 141.216) (end 66.496 140.57105) (width 0.2) (layer "B.Cu") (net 6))
 (segment (start 69.036 98.764) (end 73.5 94.3) (width 0.2) (layer "B.Cu") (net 6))
 (segment (start 62.855 140.115) (end 63.956 141.216) (width 0.2) (layer "B.Cu") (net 6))
 (segment (start 63.956 141.216) (end 65.85105 141.216) (width 0.2) (layer "B.Cu") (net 6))
 (segment (start 66.496 140.57105) (end 66.496 139.65895) (width 0.2) (layer "B.Cu") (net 6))
 (segment (start 89.5 91.5) (end 78.32 91.5) (width 0.2) (layer "F.Cu") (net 9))
 (segment (start 92.04 91.5) (end 89.5 91.5) (width 0.2) (layer "F.Cu") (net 9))
 (segment (start 78.32 91.5) (end 73.5 86.68) (width 0.2) (layer "F.Cu") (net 9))
 (segment (start 50.724 138.144) (end 52.695 140.115) (width 0.2) (layer "B.Cu") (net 9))
 (segment (start 50.724 109.456) (end 50.724 138.144) (width 0.2) (layer "B.Cu") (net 9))
 (segment (start 73.5 86.68) (end 50.724 109.456) (width 0.2) (layer "B.Cu") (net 9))
 (segment (start 90.795 138.98363) (end 90.795 140.115) (width 0.2) (layer "F.Cu") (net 1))
 (segment (start 79.534 113.034) (end 79.534 127.72263) (width 0.2) (layer "F.Cu") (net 1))
 (segment (start 73.5 107) (end 79.534 113.034) (width 0.2) (layer "F.Cu") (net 1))
 (segment (start 79.534 127.72263) (end 90.795 138.98363) (width 0.2) (layer "F.Cu") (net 1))
 (segment (start 73.5 107) (end 86.7 107) (width 0.2) (layer "B.Cu") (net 1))
 (segment (start 86.7 107) (end 89.5 104.2) (width 0.2) (layer "B.Cu") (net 1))
 (segment (start 89.5 104.2) (end 92.04 104.2) (width 0.2) (layer "B.Cu") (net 1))
 (segment (start 52.695 117.645) (end 52.695 122.335) (width 0.2) (layer "F.Cu") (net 5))
 (segment (start 73.5 96.84) (end 52.695 117.645) (width 0.2) (layer "F.Cu") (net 5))
 (segment (start 55.235 122.335) (end 55.235 117.645) (width 0.2) (layer "F.Cu") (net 4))
 (segment (start 55.235 117.645) (end 73.5 99.38) (width 0.2) (layer "F.Cu") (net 4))
 (segment (start 60.315 122.335) (end 60.315 115.105) (width 0.2) (layer "F.Cu") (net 3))
 (segment (start 60.315 115.105) (end 73.5 101.92) (width 0.2) (layer "F.Cu") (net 3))
 (segment (start 89.5 99.12) (end 92.04 99.12) (width 0.2) (layer "F.Cu") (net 16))
 (segment (start 85.311 103.309) (end 89.5 99.12) (width 0.2) (layer "F.Cu") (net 16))
 (segment (start 62.855 122.335) (end 62.855 113.47724) (width 0.2) (layer "F.Cu") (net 16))
 (segment (start 62.855 113.47724) (end 73.02324 103.309) (width 0.2) (layer "F.Cu") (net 16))
 (segment (start 73.02324 103.309) (end 85.311 103.309) (width 0.2) (layer "F.Cu") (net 16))
 (segment (start 50.224 134.217933) (end 55.015067 139.009) (width 0.2) (layer "F.Cu") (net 7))
 (segment (start 55.015067 139.009) (end 59.209 139.009) (width 0.2) (layer "F.Cu") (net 7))
 (segment (start 59.209 139.009) (end 60.315 140.115) (width 0.2) (layer "F.Cu") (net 7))
 (segment (start 89.5 94.04) (end 92.04 94.04) (width 0.2) (layer "F.Cu") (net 7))
 (segment (start 73.5 91.76) (end 75.78 94.04) (width 0.2) (layer "F.Cu") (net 7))
 (segment (start 50.224 115.036) (end 50.224 134.217933) (width 0.2) (layer "F.Cu") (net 7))
 (segment (start 75.78 94.04) (end 89.5 94.04) (width 0.2) (layer "F.Cu") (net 7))
 (segment (start 73.5 91.76) (end 50.224 115.036) (width 0.2) (layer "F.Cu") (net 7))
 (segment (start 98.415 146.195) (end 105.79 153.57) (width 0.2) (layer "F.Cu") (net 10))
 (segment (start 98.415 140.115) (end 98.415 146.195) (width 0.2) (layer "F.Cu") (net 10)))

